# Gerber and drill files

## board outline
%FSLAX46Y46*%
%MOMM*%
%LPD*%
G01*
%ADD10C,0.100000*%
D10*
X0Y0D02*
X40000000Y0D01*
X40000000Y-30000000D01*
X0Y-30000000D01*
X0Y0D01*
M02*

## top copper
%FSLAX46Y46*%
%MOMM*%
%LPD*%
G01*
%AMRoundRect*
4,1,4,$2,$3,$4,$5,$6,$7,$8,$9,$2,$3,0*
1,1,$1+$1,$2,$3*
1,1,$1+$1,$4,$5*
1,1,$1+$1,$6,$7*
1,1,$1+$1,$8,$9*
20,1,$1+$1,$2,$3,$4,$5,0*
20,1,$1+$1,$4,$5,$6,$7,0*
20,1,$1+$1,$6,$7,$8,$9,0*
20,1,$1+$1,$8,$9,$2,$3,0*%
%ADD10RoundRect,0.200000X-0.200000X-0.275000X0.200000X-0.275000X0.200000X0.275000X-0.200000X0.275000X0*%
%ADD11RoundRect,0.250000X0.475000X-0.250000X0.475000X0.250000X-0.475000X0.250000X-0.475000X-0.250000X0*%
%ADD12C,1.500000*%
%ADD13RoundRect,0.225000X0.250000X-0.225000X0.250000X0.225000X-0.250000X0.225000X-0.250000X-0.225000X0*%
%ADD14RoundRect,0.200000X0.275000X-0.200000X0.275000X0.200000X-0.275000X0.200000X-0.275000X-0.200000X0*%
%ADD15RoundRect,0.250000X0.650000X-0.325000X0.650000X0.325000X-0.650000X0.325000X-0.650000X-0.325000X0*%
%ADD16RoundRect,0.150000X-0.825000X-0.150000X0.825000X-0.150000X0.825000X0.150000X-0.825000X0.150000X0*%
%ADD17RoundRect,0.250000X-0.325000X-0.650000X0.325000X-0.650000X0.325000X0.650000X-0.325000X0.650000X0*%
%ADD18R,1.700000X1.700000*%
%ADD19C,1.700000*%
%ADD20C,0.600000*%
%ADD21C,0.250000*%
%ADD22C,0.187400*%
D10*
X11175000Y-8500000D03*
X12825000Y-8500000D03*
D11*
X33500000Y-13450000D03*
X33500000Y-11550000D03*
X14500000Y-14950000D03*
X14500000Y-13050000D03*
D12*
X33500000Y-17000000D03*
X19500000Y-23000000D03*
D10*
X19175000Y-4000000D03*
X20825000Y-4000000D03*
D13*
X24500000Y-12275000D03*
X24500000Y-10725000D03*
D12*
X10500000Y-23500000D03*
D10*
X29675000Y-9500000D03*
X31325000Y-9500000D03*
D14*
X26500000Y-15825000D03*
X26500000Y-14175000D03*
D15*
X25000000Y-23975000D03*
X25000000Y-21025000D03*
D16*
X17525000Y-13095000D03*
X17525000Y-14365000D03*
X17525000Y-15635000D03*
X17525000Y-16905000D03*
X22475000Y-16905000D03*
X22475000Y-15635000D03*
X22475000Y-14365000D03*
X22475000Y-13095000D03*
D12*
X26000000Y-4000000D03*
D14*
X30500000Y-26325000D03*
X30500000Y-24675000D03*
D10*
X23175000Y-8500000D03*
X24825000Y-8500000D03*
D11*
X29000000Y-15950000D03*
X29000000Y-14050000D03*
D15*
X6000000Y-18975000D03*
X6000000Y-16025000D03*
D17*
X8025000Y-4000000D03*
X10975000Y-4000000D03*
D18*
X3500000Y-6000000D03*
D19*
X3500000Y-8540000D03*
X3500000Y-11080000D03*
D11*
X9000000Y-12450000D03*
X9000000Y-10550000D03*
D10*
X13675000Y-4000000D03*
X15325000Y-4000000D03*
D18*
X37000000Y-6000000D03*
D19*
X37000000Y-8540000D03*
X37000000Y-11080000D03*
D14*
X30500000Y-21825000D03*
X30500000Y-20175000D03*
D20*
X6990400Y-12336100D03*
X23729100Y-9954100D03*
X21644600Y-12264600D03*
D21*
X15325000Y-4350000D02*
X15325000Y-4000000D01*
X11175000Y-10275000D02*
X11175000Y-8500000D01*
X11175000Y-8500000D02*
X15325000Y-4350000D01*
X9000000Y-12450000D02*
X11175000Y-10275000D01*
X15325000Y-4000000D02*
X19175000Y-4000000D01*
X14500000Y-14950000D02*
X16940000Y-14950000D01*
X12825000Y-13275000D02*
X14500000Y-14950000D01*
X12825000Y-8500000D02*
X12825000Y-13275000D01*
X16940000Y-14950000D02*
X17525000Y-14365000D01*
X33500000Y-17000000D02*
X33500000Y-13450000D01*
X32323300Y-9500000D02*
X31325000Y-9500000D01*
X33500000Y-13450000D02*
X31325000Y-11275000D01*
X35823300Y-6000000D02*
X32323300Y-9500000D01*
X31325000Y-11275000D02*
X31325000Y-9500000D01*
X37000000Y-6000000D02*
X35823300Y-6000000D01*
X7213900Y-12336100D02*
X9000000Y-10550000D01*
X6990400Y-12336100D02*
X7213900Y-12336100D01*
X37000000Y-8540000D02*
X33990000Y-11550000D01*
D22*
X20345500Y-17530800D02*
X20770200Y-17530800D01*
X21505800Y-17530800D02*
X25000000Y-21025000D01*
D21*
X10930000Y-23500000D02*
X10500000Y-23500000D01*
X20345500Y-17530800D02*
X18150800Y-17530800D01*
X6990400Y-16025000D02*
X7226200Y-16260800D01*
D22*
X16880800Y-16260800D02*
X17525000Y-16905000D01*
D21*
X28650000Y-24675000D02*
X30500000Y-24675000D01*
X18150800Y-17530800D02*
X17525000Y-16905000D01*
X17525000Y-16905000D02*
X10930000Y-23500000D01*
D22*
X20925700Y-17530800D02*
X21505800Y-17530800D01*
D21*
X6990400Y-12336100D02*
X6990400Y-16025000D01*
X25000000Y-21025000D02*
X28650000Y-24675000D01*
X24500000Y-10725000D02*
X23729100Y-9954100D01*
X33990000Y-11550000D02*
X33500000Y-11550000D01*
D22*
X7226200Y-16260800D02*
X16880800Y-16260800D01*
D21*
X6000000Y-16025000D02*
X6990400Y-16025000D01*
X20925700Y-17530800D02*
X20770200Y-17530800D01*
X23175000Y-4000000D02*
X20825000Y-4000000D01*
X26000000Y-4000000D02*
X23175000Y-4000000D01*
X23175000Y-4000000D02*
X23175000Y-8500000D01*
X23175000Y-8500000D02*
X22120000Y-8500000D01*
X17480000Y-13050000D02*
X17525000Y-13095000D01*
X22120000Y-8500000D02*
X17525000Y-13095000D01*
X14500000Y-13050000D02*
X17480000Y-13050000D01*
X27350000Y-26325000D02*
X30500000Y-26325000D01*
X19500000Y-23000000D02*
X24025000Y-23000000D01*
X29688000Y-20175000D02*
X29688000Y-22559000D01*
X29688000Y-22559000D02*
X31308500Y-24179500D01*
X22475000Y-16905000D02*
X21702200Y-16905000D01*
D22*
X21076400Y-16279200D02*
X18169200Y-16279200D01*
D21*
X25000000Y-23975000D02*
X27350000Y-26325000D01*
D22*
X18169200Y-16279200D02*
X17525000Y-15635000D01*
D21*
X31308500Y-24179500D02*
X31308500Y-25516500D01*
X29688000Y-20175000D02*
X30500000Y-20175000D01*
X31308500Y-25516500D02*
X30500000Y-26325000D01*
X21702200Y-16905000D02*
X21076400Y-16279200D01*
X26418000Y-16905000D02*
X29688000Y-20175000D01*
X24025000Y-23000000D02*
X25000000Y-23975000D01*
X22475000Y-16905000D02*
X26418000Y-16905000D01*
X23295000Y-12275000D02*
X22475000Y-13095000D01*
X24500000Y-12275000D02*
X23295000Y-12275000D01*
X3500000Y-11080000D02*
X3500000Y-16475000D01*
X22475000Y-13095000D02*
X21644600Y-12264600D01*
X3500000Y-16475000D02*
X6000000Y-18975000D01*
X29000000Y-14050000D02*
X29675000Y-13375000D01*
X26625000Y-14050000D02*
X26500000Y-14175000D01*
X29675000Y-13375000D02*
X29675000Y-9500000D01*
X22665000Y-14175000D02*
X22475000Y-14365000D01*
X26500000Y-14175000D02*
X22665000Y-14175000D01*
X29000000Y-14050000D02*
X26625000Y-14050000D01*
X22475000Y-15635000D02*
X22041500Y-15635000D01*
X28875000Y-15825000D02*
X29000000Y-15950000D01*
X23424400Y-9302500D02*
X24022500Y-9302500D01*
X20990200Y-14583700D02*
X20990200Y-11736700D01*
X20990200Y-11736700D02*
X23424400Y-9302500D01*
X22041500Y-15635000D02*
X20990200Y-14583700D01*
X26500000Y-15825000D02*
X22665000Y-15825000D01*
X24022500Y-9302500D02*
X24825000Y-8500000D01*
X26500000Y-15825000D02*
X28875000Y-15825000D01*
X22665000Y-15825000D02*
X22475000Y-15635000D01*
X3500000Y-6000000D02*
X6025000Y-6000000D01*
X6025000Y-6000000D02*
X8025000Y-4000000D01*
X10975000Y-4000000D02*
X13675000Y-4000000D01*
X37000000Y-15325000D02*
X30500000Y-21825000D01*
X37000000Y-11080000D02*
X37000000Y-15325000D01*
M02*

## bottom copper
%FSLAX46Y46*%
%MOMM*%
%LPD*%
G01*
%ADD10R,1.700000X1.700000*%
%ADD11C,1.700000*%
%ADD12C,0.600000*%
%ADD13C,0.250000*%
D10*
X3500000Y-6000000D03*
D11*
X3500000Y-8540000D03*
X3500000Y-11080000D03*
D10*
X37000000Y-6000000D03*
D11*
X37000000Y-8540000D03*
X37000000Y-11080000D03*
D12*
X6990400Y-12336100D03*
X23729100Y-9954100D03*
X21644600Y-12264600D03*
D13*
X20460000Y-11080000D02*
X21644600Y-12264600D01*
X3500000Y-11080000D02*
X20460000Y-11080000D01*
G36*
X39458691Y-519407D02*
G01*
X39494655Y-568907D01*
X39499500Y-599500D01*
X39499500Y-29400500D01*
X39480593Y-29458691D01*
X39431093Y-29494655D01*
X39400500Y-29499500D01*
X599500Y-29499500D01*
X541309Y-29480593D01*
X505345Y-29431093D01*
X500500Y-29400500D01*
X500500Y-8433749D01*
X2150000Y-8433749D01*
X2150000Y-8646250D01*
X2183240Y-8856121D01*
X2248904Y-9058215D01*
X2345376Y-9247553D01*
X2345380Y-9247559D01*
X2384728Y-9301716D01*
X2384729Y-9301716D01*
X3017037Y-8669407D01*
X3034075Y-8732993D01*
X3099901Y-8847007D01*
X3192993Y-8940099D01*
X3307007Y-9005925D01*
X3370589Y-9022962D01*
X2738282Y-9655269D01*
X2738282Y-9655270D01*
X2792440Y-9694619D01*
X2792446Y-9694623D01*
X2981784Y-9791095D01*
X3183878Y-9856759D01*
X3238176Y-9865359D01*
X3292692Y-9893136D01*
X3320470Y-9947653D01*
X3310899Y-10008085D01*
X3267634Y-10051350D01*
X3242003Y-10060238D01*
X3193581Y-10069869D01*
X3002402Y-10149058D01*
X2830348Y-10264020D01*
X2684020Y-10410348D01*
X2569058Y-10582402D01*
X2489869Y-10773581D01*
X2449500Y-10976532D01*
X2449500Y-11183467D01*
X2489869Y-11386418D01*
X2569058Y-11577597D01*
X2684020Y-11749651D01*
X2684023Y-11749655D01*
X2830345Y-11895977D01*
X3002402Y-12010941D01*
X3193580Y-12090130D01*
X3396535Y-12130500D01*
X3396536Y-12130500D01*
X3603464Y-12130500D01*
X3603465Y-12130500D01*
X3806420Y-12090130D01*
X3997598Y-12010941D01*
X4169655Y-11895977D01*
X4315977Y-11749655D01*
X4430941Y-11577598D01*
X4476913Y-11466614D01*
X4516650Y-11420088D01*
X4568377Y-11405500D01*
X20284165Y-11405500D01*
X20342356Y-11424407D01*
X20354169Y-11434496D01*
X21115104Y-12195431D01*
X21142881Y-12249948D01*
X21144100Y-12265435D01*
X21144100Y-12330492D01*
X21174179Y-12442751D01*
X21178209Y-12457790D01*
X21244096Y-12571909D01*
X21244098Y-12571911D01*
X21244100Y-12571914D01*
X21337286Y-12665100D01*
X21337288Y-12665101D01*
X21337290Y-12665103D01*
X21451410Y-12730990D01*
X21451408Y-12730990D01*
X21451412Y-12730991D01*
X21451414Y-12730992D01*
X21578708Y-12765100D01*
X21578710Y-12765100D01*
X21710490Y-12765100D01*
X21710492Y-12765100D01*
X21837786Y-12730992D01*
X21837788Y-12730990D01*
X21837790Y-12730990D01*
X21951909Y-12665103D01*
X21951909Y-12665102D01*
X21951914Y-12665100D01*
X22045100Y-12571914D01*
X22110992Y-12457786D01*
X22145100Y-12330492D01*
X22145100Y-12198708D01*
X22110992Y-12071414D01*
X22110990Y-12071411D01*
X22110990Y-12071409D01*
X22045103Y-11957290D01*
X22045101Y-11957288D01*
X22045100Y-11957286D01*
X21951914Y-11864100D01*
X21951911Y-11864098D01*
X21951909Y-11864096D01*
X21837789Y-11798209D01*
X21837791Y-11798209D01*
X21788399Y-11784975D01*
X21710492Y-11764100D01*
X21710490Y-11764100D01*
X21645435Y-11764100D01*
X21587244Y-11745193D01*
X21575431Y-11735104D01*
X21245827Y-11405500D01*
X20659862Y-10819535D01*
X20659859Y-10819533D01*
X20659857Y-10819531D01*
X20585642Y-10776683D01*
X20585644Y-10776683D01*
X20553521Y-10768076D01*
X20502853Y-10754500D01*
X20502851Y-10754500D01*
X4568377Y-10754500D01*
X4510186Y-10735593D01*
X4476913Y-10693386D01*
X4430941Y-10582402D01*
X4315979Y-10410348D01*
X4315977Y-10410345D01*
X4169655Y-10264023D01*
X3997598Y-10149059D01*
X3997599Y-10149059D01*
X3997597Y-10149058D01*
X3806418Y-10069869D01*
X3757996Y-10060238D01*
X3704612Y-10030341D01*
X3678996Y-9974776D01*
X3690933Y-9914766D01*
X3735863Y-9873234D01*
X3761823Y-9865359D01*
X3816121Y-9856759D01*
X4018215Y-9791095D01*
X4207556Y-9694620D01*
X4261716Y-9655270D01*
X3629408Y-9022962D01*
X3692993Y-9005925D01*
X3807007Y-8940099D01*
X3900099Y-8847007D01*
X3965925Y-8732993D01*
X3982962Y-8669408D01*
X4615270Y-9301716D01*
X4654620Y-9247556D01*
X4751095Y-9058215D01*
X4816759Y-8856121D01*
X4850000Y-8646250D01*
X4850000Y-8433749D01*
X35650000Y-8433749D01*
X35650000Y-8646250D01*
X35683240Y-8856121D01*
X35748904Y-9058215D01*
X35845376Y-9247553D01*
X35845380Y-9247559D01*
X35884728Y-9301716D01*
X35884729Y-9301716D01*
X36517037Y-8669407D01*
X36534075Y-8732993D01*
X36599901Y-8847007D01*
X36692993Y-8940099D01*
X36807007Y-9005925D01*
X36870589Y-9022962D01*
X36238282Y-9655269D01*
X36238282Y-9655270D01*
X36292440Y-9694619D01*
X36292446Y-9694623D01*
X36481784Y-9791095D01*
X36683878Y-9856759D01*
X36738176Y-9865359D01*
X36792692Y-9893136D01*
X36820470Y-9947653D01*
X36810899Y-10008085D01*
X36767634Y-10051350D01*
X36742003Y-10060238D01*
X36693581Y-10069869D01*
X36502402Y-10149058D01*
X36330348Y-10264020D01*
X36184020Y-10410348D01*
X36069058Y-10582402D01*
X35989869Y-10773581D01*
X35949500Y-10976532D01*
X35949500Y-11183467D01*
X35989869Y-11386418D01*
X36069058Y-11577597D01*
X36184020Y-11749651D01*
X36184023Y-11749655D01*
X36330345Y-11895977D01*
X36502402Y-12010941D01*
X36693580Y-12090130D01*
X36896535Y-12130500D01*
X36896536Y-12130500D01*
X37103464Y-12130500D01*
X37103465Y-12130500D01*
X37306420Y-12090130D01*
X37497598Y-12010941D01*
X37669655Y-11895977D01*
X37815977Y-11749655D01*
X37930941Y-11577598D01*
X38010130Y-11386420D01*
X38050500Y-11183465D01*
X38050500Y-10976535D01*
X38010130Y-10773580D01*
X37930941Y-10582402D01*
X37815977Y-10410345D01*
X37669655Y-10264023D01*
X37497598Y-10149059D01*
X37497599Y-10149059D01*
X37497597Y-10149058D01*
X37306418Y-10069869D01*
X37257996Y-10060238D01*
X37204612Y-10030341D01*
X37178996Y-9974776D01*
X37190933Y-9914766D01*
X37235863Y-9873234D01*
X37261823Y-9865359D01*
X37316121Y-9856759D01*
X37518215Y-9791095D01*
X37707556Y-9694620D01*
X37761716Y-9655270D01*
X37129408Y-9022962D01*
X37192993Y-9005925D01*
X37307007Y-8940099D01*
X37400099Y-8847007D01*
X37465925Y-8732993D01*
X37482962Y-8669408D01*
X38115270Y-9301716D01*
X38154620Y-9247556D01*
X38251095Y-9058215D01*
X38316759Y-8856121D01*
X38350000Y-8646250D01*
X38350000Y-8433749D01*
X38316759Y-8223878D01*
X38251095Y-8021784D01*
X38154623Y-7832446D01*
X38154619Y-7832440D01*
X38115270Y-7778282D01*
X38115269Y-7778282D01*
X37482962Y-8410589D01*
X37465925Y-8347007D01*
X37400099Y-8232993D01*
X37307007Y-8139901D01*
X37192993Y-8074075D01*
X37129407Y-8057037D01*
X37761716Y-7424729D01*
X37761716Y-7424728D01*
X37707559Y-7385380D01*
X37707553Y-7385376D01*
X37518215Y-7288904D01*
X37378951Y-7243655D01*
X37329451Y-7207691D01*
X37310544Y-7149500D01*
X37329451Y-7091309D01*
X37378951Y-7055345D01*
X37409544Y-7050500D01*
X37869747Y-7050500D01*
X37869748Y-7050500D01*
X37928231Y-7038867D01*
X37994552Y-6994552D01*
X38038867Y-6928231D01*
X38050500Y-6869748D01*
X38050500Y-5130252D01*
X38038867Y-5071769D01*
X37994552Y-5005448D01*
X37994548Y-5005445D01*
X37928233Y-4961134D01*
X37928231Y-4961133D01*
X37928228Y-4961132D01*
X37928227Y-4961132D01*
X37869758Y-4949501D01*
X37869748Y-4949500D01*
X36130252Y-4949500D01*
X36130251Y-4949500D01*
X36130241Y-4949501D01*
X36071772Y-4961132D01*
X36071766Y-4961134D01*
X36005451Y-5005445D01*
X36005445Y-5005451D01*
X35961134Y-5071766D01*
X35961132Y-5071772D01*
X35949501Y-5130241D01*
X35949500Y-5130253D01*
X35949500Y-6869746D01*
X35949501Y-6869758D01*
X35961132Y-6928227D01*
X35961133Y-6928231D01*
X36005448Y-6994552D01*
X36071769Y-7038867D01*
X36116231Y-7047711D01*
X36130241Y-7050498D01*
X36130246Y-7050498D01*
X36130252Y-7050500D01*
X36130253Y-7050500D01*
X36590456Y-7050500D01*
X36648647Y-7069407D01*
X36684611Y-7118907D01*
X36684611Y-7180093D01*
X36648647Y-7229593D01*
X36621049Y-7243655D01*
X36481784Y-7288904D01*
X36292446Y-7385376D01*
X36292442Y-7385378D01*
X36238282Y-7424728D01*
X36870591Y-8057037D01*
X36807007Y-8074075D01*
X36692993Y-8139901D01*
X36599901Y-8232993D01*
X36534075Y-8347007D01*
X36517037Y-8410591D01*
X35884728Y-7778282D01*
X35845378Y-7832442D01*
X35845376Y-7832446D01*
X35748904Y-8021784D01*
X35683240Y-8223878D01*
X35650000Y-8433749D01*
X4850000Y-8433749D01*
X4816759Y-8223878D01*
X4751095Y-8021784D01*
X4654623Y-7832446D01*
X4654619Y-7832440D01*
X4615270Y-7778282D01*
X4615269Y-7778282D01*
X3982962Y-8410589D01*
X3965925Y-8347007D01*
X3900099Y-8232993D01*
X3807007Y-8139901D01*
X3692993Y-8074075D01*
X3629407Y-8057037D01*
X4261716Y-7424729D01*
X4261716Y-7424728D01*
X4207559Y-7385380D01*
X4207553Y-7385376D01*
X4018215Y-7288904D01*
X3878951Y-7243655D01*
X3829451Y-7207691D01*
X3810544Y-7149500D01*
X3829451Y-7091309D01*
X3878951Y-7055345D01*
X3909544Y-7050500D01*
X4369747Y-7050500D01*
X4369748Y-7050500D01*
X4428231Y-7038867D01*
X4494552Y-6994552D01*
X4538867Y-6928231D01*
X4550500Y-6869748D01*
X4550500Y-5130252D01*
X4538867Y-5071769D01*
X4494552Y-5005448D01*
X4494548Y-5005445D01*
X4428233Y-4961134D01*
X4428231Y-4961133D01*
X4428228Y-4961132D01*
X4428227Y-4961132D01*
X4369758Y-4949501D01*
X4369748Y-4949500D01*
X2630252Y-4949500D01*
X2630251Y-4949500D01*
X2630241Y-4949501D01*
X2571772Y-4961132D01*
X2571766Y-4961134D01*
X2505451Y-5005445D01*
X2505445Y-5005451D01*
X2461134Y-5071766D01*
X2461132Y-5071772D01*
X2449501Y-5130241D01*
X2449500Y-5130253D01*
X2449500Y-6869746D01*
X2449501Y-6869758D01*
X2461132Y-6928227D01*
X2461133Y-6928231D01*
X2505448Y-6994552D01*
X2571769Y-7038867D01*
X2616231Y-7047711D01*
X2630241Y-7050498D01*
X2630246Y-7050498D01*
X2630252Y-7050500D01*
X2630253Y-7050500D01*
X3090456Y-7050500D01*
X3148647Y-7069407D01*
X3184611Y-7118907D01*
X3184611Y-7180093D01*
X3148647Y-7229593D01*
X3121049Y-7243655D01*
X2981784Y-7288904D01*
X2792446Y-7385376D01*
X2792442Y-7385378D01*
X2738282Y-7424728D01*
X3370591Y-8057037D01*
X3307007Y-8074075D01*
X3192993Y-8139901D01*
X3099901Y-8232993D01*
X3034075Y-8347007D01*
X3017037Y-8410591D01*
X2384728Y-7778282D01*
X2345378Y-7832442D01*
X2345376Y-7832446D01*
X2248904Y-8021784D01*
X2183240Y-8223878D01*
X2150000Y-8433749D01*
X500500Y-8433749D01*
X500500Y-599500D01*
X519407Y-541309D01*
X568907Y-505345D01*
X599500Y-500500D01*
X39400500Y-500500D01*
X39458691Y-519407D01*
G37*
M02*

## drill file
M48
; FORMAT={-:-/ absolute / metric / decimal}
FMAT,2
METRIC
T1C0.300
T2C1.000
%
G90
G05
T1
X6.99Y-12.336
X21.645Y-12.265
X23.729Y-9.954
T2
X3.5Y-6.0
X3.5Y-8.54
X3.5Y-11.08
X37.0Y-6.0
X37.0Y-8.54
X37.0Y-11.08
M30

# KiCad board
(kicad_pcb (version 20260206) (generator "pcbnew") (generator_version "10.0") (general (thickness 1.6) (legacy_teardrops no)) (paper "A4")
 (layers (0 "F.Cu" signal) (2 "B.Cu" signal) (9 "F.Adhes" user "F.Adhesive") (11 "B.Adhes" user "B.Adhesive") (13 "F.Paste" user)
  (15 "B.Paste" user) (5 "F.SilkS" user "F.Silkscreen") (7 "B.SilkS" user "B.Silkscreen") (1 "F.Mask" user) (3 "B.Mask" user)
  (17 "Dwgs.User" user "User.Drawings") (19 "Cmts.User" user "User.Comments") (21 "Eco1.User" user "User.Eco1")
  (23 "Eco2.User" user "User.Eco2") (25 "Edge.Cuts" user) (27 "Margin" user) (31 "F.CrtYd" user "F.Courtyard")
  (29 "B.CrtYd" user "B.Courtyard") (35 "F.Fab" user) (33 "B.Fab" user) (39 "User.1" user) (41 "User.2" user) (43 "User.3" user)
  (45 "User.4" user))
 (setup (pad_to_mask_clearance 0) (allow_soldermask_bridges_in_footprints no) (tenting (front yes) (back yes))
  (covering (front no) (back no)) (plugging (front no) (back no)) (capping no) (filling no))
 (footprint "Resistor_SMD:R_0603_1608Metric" (layer "F.Cu") (at 12 8.5)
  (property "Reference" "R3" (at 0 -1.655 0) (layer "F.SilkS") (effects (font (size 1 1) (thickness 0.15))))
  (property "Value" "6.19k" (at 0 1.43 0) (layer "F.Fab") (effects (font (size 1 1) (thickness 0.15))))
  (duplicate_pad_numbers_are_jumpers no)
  (pad "1" smd roundrect (at -0.825 0) (size 0.8 0.95) (layers "F.Cu" "F.Mask" "F.Paste") (roundrect_rratio 0.25) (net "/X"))
  (pad "2" smd roundrect (at 0.825 0) (size 0.8 0.95) (layers "F.Cu" "F.Mask" "F.Paste") (roundrect_rratio 0.25) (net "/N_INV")))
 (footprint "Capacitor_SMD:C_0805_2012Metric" (layer "F.Cu") (at 33.5 12.5 90)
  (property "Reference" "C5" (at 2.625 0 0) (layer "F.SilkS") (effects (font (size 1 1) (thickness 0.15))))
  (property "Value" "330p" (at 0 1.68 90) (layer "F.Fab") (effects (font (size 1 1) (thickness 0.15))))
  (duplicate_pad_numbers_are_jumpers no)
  (pad "1" smd roundrect (at -0.95 0 90) (size 1 1.45) (layers "F.Cu" "F.Mask" "F.Paste") (roundrect_rratio 0.25) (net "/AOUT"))
  (pad "2" smd roundrect (at 0.95 0 90) (size 1 1.45) (layers "F.Cu" "F.Mask" "F.Paste") (roundrect_rratio 0.25) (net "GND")))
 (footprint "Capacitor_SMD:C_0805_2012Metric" (layer "F.Cu") (at 14.5 14 90)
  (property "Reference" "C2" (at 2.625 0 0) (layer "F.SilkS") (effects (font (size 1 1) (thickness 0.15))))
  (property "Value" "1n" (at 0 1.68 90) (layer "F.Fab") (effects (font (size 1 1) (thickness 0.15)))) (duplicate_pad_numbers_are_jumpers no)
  (pad "1" smd roundrect (at -0.95 0 90) (size 1 1.45) (layers "F.Cu" "F.Mask" "F.Paste") (roundrect_rratio 0.25) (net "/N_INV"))
  (pad "2" smd roundrect (at 0.95 0 90) (size 1 1.45) (layers "F.Cu" "F.Mask" "F.Paste") (roundrect_rratio 0.25) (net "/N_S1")))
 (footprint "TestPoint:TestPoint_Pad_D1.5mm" (layer "F.Cu") (at 33.5 17)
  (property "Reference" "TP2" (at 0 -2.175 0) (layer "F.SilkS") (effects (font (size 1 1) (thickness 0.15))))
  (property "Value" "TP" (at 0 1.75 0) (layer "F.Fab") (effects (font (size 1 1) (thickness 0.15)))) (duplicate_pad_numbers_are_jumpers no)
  (pad "1" smd circle (at 0 0) (size 1.5 1.5) (layers "F.Cu" "F.Mask") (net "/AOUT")))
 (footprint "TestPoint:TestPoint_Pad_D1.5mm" (layer "F.Cu") (at 19.5 23)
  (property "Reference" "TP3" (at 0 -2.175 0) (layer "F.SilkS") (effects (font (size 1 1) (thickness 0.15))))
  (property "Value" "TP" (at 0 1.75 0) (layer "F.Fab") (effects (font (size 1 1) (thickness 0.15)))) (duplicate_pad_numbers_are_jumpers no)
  (pad "1" smd circle (at 0 0) (size 1.5 1.5) (layers "F.Cu" "F.Mask") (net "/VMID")))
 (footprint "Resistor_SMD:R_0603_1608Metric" (layer "F.Cu") (at 20 4)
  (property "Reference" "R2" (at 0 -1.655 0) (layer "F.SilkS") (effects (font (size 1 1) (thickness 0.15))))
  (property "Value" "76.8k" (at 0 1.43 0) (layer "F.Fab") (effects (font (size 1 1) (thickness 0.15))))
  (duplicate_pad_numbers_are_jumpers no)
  (pad "1" smd roundrect (at -0.825 0) (size 0.8 0.95) (layers "F.Cu" "F.Mask" "F.Paste") (roundrect_rratio 0.25) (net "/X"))
  (pad "2" smd roundrect (at 0.825 0) (size 0.8 0.95) (layers "F.Cu" "F.Mask" "F.Paste") (roundrect_rratio 0.25) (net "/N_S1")))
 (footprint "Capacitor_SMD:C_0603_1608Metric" (layer "F.Cu") (at 24.5 11.5 90)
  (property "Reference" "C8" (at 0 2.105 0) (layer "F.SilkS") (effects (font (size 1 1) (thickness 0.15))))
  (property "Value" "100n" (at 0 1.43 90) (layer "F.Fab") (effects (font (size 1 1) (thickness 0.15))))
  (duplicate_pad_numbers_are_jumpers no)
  (pad "1" smd roundrect (at -0.775 0 90) (size 0.9 0.95) (layers "F.Cu" "F.Mask" "F.Paste") (roundrect_rratio 0.25) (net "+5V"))
  (pad "2" smd roundrect (at 0.775 0 90) (size 0.9 0.95) (layers "F.Cu" "F.Mask" "F.Paste") (roundrect_rratio 0.25) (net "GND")))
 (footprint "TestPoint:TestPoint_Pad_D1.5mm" (layer "F.Cu") (at 10.5 23.5)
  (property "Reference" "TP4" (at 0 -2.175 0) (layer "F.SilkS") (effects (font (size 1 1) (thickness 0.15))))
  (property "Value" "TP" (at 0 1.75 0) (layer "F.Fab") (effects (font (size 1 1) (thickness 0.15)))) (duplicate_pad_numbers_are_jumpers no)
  (pad "1" smd circle (at 0 0) (size 1.5 1.5) (layers "F.Cu" "F.Mask") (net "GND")))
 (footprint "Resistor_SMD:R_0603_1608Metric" (layer "F.Cu") (at 30.5 9.5)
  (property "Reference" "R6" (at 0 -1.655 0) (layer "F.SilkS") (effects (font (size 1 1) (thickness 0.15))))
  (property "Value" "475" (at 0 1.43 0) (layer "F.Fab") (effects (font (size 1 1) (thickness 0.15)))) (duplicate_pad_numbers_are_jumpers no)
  (pad "1" smd roundrect (at -0.825 0) (size 0.8 0.95) (layers "F.Cu" "F.Mask" "F.Paste") (roundrect_rratio 0.25) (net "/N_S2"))
  (pad "2" smd roundrect (at 0.825 0) (size 0.8 0.95) (layers "F.Cu" "F.Mask" "F.Paste") (roundrect_rratio 0.25) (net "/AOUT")))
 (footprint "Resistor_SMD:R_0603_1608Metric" (layer "F.Cu") (at 26.5 15 90)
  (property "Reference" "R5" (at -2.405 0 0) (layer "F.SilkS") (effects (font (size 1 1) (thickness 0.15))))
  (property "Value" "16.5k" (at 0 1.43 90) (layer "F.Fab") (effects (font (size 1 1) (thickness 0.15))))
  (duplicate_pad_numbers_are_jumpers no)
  (pad "1" smd roundrect (at -0.825 0 90) (size 0.8 0.95) (layers "F.Cu" "F.Mask" "F.Paste") (roundrect_rratio 0.25) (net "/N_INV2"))
  (pad "2" smd roundrect (at 0.825 0 90) (size 0.8 0.95) (layers "F.Cu" "F.Mask" "F.Paste") (roundrect_rratio 0.25) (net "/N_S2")))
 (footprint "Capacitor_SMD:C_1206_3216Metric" (layer "F.Cu") (at 25 22.5 90)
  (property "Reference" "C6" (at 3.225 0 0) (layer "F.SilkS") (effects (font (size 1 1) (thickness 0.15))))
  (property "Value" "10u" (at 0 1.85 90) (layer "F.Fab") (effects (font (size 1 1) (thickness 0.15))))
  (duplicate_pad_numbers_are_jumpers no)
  (pad "1" smd roundrect (at -1.475 0 90) (size 1.15 1.8) (layers "F.Cu" "F.Mask" "F.Paste") (roundrect_rratio 0.217391) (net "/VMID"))
  (pad "2" smd roundrect (at 1.475 0 90) (size 1.15 1.8) (layers "F.Cu" "F.Mask" "F.Paste") (roundrect_rratio 0.217391) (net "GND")))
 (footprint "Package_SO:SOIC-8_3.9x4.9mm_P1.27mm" (layer "F.Cu") (at 20 15)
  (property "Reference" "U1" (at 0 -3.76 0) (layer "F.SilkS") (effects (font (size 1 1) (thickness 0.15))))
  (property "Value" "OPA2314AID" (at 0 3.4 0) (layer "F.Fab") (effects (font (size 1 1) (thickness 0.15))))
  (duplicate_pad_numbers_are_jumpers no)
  (pad "1" smd roundrect (at -2.475 -1.905) (size 1.95 0.6) (layers "F.Cu" "F.Mask" "F.Paste") (roundrect_rratio 0.25) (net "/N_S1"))
  (pad "2" smd roundrect (at -2.475 -0.635) (size 1.95 0.6) (layers "F.Cu" "F.Mask" "F.Paste") (roundrect_rratio 0.25) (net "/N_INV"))
  (pad "3" smd roundrect (at -2.475 0.635) (size 1.95 0.6) (layers "F.Cu" "F.Mask" "F.Paste") (roundrect_rratio 0.25) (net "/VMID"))
  (pad "4" smd roundrect (at -2.475 1.905) (size 1.95 0.6) (layers "F.Cu" "F.Mask" "F.Paste") (roundrect_rratio 0.25) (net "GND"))
  (pad "5" smd roundrect (at 2.475 1.905) (size 1.95 0.6) (layers "F.Cu" "F.Mask" "F.Paste") (roundrect_rratio 0.25) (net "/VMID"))
  (pad "6" smd roundrect (at 2.475 0.635) (size 1.95 0.6) (layers "F.Cu" "F.Mask" "F.Paste") (roundrect_rratio 0.25) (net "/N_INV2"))
  (pad "7" smd roundrect (at 2.475 -0.635) (size 1.95 0.6) (layers "F.Cu" "F.Mask" "F.Paste") (roundrect_rratio 0.25) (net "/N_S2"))
  (pad "8" smd roundrect (at 2.475 -1.905) (size 1.95 0.6) (layers "F.Cu" "F.Mask" "F.Paste") (roundrect_rratio 0.25) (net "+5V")))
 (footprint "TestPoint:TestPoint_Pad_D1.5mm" (layer "F.Cu") (at 26 4)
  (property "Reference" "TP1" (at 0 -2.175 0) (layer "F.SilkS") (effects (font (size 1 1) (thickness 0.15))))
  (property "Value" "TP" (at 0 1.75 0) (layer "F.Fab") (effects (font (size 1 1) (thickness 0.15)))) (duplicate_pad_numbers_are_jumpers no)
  (pad "1" smd circle (at 0 0) (size 1.5 1.5) (layers "F.Cu" "F.Mask") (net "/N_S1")))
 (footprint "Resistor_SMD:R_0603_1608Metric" (layer "F.Cu") (at 30.5 25.5 90)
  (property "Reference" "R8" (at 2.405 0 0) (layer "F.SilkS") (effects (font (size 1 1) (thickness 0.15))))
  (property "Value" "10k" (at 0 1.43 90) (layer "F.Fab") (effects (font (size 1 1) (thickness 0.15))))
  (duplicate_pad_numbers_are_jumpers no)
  (pad "1" smd roundrect (at -0.825 0 90) (size 0.8 0.95) (layers "F.Cu" "F.Mask" "F.Paste") (roundrect_rratio 0.25) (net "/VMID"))
  (pad "2" smd roundrect (at 0.825 0 90) (size 0.8 0.95) (layers "F.Cu" "F.Mask" "F.Paste") (roundrect_rratio 0.25) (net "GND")))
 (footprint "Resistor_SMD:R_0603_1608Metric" (layer "F.Cu") (at 24 8.5)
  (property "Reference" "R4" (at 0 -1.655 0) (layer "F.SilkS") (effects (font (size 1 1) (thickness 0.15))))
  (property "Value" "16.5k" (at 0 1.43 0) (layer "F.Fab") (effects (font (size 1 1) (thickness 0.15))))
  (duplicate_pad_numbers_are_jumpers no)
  (pad "1" smd roundrect (at -0.825 0) (size 0.8 0.95) (layers "F.Cu" "F.Mask" "F.Paste") (roundrect_rratio 0.25) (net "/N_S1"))
  (pad "2" smd roundrect (at 0.825 0) (size 0.8 0.95) (layers "F.Cu" "F.Mask" "F.Paste") (roundrect_rratio 0.25) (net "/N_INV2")))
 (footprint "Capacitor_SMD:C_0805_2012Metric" (layer "F.Cu") (at 29 15 90)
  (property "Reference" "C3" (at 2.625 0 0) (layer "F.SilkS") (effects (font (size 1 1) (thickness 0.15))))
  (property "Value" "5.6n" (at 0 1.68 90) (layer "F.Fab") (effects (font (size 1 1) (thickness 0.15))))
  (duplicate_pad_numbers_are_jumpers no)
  (pad "1" smd roundrect (at -0.95 0 90) (size 1 1.45) (layers "F.Cu" "F.Mask" "F.Paste") (roundrect_rratio 0.25) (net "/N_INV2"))
  (pad "2" smd roundrect (at 0.95 0 90) (size 1 1.45) (layers "F.Cu" "F.Mask" "F.Paste") (roundrect_rratio 0.25) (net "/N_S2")))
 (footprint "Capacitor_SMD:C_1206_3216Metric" (layer "F.Cu") (at 6 17.5 90)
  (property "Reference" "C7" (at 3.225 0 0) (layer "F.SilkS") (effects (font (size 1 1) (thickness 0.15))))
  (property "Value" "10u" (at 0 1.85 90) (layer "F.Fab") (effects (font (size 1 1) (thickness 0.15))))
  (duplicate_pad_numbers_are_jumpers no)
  (pad "1" smd roundrect (at -1.475 0 90) (size 1.15 1.8) (layers "F.Cu" "F.Mask" "F.Paste") (roundrect_rratio 0.217391) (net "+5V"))
  (pad "2" smd roundrect (at 1.475 0 90) (size 1.15 1.8) (layers "F.Cu" "F.Mask" "F.Paste") (roundrect_rratio 0.217391) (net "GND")))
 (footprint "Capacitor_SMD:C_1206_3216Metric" (layer "F.Cu") (at 9.5 4)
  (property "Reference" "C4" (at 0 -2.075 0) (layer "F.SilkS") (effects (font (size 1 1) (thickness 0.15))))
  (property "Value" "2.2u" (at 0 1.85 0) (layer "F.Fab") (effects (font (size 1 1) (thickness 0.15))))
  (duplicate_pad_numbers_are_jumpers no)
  (pad "1" smd roundrect (at -1.475 0) (size 1.15 1.8) (layers "F.Cu" "F.Mask" "F.Paste") (roundrect_rratio 0.217391) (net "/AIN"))
  (pad "2" smd roundrect (at 1.475 0) (size 1.15 1.8) (layers "F.Cu" "F.Mask" "F.Paste") (roundrect_rratio 0.217391) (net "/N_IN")))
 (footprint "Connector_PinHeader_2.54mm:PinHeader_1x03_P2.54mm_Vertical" (layer "F.Cu") (at 3.5 6)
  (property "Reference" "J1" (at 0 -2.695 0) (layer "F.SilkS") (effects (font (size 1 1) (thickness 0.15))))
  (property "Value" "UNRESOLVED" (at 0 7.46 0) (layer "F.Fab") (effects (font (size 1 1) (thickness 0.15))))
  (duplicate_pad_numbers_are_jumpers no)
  (pad "1" thru_hole rect (at 0 0) (size 1.7 1.7) (drill 1) (layers "*.Cu" "*.Mask") (remove_unused_layers no) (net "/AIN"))
  (pad "2" thru_hole circle (at 0 2.54) (size 1.7 1.7) (drill 1) (layers "*.Cu" "*.Mask") (remove_unused_layers no) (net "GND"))
  (pad "3" thru_hole circle (at 0 5.08) (size 1.7 1.7) (drill 1) (layers "*.Cu" "*.Mask") (remove_unused_layers no) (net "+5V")))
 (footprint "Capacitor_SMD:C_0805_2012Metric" (layer "F.Cu") (at 9 11.5 90)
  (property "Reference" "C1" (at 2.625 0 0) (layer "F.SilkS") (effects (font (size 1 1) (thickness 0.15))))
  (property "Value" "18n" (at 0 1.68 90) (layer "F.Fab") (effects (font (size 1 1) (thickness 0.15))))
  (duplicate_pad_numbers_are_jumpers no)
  (pad "1" smd roundrect (at -0.95 0 90) (size 1 1.45) (layers "F.Cu" "F.Mask" "F.Paste") (roundrect_rratio 0.25) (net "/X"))
  (pad "2" smd roundrect (at 0.95 0 90) (size 1 1.45) (layers "F.Cu" "F.Mask" "F.Paste") (roundrect_rratio 0.25) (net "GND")))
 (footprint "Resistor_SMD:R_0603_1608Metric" (layer "F.Cu") (at 14.5 4)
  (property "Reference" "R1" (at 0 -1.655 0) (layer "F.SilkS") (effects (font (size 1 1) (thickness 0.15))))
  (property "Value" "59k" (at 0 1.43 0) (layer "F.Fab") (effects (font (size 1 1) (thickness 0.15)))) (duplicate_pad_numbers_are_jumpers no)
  (pad "1" smd roundrect (at -0.825 0) (size 0.8 0.95) (layers "F.Cu" "F.Mask" "F.Paste") (roundrect_rratio 0.25) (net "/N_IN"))
  (pad "2" smd roundrect (at 0.825 0) (size 0.8 0.95) (layers "F.Cu" "F.Mask" "F.Paste") (roundrect_rratio 0.25) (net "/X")))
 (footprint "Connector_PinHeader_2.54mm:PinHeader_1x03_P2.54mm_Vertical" (layer "F.Cu") (at 37 6)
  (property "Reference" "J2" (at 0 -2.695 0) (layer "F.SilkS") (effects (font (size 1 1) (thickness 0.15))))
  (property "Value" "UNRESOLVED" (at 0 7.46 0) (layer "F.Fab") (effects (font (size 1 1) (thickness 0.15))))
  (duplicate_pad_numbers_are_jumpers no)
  (pad "1" thru_hole rect (at 0 0) (size 1.7 1.7) (drill 1) (layers "*.Cu" "*.Mask") (remove_unused_layers no) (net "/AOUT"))
  (pad "2" thru_hole circle (at 0 2.54) (size 1.7 1.7) (drill 1) (layers "*.Cu" "*.Mask") (remove_unused_layers no) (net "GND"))
  (pad "3" thru_hole circle (at 0 5.08) (size 1.7 1.7) (drill 1) (layers "*.Cu" "*.Mask") (remove_unused_layers no) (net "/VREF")))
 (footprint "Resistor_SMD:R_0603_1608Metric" (layer "F.Cu") (at 30.5 21 90)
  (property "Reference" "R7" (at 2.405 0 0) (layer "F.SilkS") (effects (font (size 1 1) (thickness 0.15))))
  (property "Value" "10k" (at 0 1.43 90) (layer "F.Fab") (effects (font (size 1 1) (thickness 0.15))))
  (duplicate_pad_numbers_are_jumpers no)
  (pad "1" smd roundrect (at -0.825 0 90) (size 0.8 0.95) (layers "F.Cu" "F.Mask" "F.Paste") (roundrect_rratio 0.25) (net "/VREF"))
  (pad "2" smd roundrect (at 0.825 0 90) (size 0.8 0.95) (layers "F.Cu" "F.Mask" "F.Paste") (roundrect_rratio 0.25) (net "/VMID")))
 (gr_rect (start 0 0) (end 40 30) (stroke (width 0.1) (type default)) (fill no) (layer "Edge.Cuts"))
 (segment (start 15.325 4.35) (end 15.325 4) (width 0.25) (layer "F.Cu") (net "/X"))
 (segment (start 11.175 10.275) (end 11.175 8.5) (width 0.25) (layer "F.Cu") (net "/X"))
 (segment (start 11.175 8.5) (end 15.325 4.35) (width 0.25) (layer "F.Cu") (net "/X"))
 (segment (start 9 12.45) (end 11.175 10.275) (width 0.25) (layer "F.Cu") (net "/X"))
 (segment (start 15.325 4) (end 19.175 4) (width 0.25) (layer "F.Cu") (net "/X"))
 (segment (start 14.5 14.95) (end 16.94 14.95) (width 0.25) (layer "F.Cu") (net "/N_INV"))
 (segment (start 12.825 13.275) (end 14.5 14.95) (width 0.25) (layer "F.Cu") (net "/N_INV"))
 (segment (start 12.825 8.5) (end 12.825 13.275) (width 0.25) (layer "F.Cu") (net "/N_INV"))
 (segment (start 16.94 14.95) (end 17.525 14.365) (width 0.25) (layer "F.Cu") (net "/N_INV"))
 (segment (start 33.5 17) (end 33.5 13.45) (width 0.25) (layer "F.Cu") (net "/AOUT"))
 (segment (start 32.3233 9.5) (end 31.325 9.5) (width 0.25) (layer "F.Cu") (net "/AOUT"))
 (segment (start 33.5 13.45) (end 31.325 11.275) (width 0.25) (layer "F.Cu") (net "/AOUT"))
 (segment (start 35.8233 6) (end 32.3233 9.5) (width 0.25) (layer "F.Cu") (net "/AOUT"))
 (segment (start 31.325 11.275) (end 31.325 9.5) (width 0.25) (layer "F.Cu") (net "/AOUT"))
 (segment (start 37 6) (end 35.8233 6) (width 0.25) (layer "F.Cu") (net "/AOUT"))
 (segment (start 7.2139 12.3361) (end 9 10.55) (width 0.25) (layer "F.Cu") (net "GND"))
 (segment (start 6.9904 12.3361) (end 7.2139 12.3361) (width 0.25) (layer "F.Cu") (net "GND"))
 (segment (start 37 8.54) (end 33.99 11.55) (width 0.25) (layer "F.Cu") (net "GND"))
 (segment (start 20.3455 17.5308) (end 20.7702 17.5308) (width 0.1874) (layer "F.Cu") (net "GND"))
 (segment (start 21.5058 17.5308) (end 25 21.025) (width 0.1874) (layer "F.Cu") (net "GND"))
 (segment (start 10.93 23.5) (end 10.5 23.5) (width 0.25) (layer "F.Cu") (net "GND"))
 (segment (start 20.3455 17.5308) (end 18.1508 17.5308) (width 0.25) (layer "F.Cu") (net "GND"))
 (segment (start 6.9904 16.025) (end 7.2262 16.2608) (width 0.25) (layer "F.Cu") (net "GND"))
 (segment (start 16.8808 16.2608) (end 17.525 16.905) (width 0.1874) (layer "F.Cu") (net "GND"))
 (segment (start 28.65 24.675) (end 30.5 24.675) (width 0.25) (layer "F.Cu") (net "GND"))
 (segment (start 18.1508 17.5308) (end 17.525 16.905) (width 0.25) (layer "F.Cu") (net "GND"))
 (segment (start 17.525 16.905) (end 10.93 23.5) (width 0.25) (layer "F.Cu") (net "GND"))
 (segment (start 20.9257 17.5308) (end 21.5058 17.5308) (width 0.1874) (layer "F.Cu") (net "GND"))
 (segment (start 6.9904 12.3361) (end 6.9904 16.025) (width 0.25) (layer "F.Cu") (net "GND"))
 (segment (start 25 21.025) (end 28.65 24.675) (width 0.25) (layer "F.Cu") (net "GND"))
 (segment (start 24.5 10.725) (end 23.7291 9.9541) (width 0.25) (layer "F.Cu") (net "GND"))
 (segment (start 33.99 11.55) (end 33.5 11.55) (width 0.25) (layer "F.Cu") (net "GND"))
 (segment (start 7.2262 16.2608) (end 16.8808 16.2608) (width 0.1874) (layer "F.Cu") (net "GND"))
 (segment (start 6 16.025) (end 6.9904 16.025) (width 0.25) (layer "F.Cu") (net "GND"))
 (segment (start 20.9257 17.5308) (end 20.7702 17.5308) (width 0.25) (layer "F.Cu") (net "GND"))
 (via (at 6.9904 12.3361) (size 0.6) (drill 0.3) (layers "F.Cu" "B.Cu") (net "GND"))
 (via (at 23.7291 9.9541) (size 0.6) (drill 0.3) (layers "F.Cu" "B.Cu") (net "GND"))
 (segment (start 23.175 4) (end 20.825 4) (width 0.25) (layer "F.Cu") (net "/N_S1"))
 (segment (start 26 4) (end 23.175 4) (width 0.25) (layer "F.Cu") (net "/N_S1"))
 (segment (start 23.175 4) (end 23.175 8.5) (width 0.25) (layer "F.Cu") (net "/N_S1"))
 (segment (start 23.175 8.5) (end 22.12 8.5) (width 0.25) (layer "F.Cu") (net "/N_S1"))
 (segment (start 17.48 13.05) (end 17.525 13.095) (width 0.25) (layer "F.Cu") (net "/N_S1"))
 (segment (start 22.12 8.5) (end 17.525 13.095) (width 0.25) (layer "F.Cu") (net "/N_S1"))
 (segment (start 14.5 13.05) (end 17.48 13.05) (width 0.25) (layer "F.Cu") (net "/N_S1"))
 (segment (start 27.35 26.325) (end 30.5 26.325) (width 0.25) (layer "F.Cu") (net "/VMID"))
 (segment (start 19.5 23) (end 24.025 23) (width 0.25) (layer "F.Cu") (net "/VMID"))
 (segment (start 29.688 20.175) (end 29.688 22.559) (width 0.25) (layer "F.Cu") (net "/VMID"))
 (segment (start 29.688 22.559) (end 31.3085 24.1795) (width 0.25) (layer "F.Cu") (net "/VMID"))
 (segment (start 22.475 16.905) (end 21.7022 16.905) (width 0.25) (layer "F.Cu") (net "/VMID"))
 (segment (start 21.0764 16.2792) (end 18.1692 16.2792) (width 0.1874) (layer "F.Cu") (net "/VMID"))
 (segment (start 25 23.975) (end 27.35 26.325) (width 0.25) (layer "F.Cu") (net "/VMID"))
 (segment (start 18.1692 16.2792) (end 17.525 15.635) (width 0.1874) (layer "F.Cu") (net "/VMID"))
 (segment (start 31.3085 24.1795) (end 31.3085 25.5165) (width 0.25) (layer "F.Cu") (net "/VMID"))
 (segment (start 29.688 20.175) (end 30.5 20.175) (width 0.25) (layer "F.Cu") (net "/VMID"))
 (segment (start 31.3085 25.5165) (end 30.5 26.325) (width 0.25) (layer "F.Cu") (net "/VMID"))
 (segment (start 21.7022 16.905) (end 21.0764 16.2792) (width 0.25) (layer "F.Cu") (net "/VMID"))
 (segment (start 26.418 16.905) (end 29.688 20.175) (width 0.25) (layer "F.Cu") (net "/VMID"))
 (segment (start 24.025 23) (end 25 23.975) (width 0.25) (layer "F.Cu") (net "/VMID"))
 (segment (start 22.475 16.905) (end 26.418 16.905) (width 0.25) (layer "F.Cu") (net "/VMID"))
 (segment (start 23.295 12.275) (end 22.475 13.095) (width 0.25) (layer "F.Cu") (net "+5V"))
 (segment (start 24.5 12.275) (end 23.295 12.275) (width 0.25) (layer "F.Cu") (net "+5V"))
 (segment (start 3.5 11.08) (end 3.5 16.475) (width 0.25) (layer "F.Cu") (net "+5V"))
 (segment (start 22.475 13.095) (end 21.6446 12.2646) (width 0.25) (layer "F.Cu") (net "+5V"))
 (segment (start 3.5 16.475) (end 6 18.975) (width 0.25) (layer "F.Cu") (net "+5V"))
 (via (at 21.6446 12.2646) (size 0.6) (drill 0.3) (layers "F.Cu" "B.Cu") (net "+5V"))
 (segment (start 20.46 11.08) (end 21.6446 12.2646) (width 0.25) (layer "B.Cu") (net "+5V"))
 (segment (start 3.5 11.08) (end 20.46 11.08) (width 0.25) (layer "B.Cu") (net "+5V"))
 (segment (start 29 14.05) (end 29.675 13.375) (width 0.25) (layer "F.Cu") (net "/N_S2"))
 (segment (start 26.625 14.05) (end 26.5 14.175) (width 0.25) (layer "F.Cu") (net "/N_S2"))
 (segment (start 29.675 13.375) (end 29.675 9.5) (width 0.25) (layer "F.Cu") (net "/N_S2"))
 (segment (start 22.665 14.175) (end 22.475 14.365) (width 0.25) (layer "F.Cu") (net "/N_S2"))
 (segment (start 26.5 14.175) (end 22.665 14.175) (width 0.25) (layer "F.Cu") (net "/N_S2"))
 (segment (start 29 14.05) (end 26.625 14.05) (width 0.25) (layer "F.Cu") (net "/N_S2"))
 (segment (start 22.475 15.635) (end 22.0415 15.635) (width 0.25) (layer "F.Cu") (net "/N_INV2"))
 (segment (start 28.875 15.825) (end 29 15.95) (width 0.25) (layer "F.Cu") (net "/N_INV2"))
 (segment (start 23.4244 9.3025) (end 24.0225 9.3025) (width 0.25) (layer "F.Cu") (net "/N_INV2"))
 (segment (start 20.9902 14.5837) (end 20.9902 11.7367) (width 0.25) (layer "F.Cu") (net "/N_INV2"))
 (segment (start 20.9902 11.7367) (end 23.4244 9.3025) (width 0.25) (layer "F.Cu") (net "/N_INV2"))
 (segment (start 22.0415 15.635) (end 20.9902 14.5837) (width 0.25) (layer "F.Cu") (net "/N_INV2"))
 (segment (start 26.5 15.825) (end 22.665 15.825) (width 0.25) (layer "F.Cu") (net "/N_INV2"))
 (segment (start 24.0225 9.3025) (end 24.825 8.5) (width 0.25) (layer "F.Cu") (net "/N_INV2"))
 (segment (start 26.5 15.825) (end 28.875 15.825) (width 0.25) (layer "F.Cu") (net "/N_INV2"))
 (segment (start 22.665 15.825) (end 22.475 15.635) (width 0.25) (layer "F.Cu") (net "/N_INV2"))
 (segment (start 3.5 6) (end 6.025 6) (width 0.25) (layer "F.Cu") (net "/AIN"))
 (segment (start 6.025 6) (end 8.025 4) (width 0.25) (layer "F.Cu") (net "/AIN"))
 (segment (start 10.975 4) (end 13.675 4) (width 0.25) (layer "F.Cu") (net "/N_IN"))
 (segment (start 37 15.325) (end 30.5 21.825) (width 0.25) (layer "F.Cu") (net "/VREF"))
 (segment (start 37 11.08) (end 37 15.325) (width 0.25) (layer "F.Cu") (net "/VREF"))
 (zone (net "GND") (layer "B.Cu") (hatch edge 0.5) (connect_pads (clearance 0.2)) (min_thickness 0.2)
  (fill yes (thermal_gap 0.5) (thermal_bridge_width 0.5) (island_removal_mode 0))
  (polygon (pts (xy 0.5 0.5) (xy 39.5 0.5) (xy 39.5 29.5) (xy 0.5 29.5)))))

